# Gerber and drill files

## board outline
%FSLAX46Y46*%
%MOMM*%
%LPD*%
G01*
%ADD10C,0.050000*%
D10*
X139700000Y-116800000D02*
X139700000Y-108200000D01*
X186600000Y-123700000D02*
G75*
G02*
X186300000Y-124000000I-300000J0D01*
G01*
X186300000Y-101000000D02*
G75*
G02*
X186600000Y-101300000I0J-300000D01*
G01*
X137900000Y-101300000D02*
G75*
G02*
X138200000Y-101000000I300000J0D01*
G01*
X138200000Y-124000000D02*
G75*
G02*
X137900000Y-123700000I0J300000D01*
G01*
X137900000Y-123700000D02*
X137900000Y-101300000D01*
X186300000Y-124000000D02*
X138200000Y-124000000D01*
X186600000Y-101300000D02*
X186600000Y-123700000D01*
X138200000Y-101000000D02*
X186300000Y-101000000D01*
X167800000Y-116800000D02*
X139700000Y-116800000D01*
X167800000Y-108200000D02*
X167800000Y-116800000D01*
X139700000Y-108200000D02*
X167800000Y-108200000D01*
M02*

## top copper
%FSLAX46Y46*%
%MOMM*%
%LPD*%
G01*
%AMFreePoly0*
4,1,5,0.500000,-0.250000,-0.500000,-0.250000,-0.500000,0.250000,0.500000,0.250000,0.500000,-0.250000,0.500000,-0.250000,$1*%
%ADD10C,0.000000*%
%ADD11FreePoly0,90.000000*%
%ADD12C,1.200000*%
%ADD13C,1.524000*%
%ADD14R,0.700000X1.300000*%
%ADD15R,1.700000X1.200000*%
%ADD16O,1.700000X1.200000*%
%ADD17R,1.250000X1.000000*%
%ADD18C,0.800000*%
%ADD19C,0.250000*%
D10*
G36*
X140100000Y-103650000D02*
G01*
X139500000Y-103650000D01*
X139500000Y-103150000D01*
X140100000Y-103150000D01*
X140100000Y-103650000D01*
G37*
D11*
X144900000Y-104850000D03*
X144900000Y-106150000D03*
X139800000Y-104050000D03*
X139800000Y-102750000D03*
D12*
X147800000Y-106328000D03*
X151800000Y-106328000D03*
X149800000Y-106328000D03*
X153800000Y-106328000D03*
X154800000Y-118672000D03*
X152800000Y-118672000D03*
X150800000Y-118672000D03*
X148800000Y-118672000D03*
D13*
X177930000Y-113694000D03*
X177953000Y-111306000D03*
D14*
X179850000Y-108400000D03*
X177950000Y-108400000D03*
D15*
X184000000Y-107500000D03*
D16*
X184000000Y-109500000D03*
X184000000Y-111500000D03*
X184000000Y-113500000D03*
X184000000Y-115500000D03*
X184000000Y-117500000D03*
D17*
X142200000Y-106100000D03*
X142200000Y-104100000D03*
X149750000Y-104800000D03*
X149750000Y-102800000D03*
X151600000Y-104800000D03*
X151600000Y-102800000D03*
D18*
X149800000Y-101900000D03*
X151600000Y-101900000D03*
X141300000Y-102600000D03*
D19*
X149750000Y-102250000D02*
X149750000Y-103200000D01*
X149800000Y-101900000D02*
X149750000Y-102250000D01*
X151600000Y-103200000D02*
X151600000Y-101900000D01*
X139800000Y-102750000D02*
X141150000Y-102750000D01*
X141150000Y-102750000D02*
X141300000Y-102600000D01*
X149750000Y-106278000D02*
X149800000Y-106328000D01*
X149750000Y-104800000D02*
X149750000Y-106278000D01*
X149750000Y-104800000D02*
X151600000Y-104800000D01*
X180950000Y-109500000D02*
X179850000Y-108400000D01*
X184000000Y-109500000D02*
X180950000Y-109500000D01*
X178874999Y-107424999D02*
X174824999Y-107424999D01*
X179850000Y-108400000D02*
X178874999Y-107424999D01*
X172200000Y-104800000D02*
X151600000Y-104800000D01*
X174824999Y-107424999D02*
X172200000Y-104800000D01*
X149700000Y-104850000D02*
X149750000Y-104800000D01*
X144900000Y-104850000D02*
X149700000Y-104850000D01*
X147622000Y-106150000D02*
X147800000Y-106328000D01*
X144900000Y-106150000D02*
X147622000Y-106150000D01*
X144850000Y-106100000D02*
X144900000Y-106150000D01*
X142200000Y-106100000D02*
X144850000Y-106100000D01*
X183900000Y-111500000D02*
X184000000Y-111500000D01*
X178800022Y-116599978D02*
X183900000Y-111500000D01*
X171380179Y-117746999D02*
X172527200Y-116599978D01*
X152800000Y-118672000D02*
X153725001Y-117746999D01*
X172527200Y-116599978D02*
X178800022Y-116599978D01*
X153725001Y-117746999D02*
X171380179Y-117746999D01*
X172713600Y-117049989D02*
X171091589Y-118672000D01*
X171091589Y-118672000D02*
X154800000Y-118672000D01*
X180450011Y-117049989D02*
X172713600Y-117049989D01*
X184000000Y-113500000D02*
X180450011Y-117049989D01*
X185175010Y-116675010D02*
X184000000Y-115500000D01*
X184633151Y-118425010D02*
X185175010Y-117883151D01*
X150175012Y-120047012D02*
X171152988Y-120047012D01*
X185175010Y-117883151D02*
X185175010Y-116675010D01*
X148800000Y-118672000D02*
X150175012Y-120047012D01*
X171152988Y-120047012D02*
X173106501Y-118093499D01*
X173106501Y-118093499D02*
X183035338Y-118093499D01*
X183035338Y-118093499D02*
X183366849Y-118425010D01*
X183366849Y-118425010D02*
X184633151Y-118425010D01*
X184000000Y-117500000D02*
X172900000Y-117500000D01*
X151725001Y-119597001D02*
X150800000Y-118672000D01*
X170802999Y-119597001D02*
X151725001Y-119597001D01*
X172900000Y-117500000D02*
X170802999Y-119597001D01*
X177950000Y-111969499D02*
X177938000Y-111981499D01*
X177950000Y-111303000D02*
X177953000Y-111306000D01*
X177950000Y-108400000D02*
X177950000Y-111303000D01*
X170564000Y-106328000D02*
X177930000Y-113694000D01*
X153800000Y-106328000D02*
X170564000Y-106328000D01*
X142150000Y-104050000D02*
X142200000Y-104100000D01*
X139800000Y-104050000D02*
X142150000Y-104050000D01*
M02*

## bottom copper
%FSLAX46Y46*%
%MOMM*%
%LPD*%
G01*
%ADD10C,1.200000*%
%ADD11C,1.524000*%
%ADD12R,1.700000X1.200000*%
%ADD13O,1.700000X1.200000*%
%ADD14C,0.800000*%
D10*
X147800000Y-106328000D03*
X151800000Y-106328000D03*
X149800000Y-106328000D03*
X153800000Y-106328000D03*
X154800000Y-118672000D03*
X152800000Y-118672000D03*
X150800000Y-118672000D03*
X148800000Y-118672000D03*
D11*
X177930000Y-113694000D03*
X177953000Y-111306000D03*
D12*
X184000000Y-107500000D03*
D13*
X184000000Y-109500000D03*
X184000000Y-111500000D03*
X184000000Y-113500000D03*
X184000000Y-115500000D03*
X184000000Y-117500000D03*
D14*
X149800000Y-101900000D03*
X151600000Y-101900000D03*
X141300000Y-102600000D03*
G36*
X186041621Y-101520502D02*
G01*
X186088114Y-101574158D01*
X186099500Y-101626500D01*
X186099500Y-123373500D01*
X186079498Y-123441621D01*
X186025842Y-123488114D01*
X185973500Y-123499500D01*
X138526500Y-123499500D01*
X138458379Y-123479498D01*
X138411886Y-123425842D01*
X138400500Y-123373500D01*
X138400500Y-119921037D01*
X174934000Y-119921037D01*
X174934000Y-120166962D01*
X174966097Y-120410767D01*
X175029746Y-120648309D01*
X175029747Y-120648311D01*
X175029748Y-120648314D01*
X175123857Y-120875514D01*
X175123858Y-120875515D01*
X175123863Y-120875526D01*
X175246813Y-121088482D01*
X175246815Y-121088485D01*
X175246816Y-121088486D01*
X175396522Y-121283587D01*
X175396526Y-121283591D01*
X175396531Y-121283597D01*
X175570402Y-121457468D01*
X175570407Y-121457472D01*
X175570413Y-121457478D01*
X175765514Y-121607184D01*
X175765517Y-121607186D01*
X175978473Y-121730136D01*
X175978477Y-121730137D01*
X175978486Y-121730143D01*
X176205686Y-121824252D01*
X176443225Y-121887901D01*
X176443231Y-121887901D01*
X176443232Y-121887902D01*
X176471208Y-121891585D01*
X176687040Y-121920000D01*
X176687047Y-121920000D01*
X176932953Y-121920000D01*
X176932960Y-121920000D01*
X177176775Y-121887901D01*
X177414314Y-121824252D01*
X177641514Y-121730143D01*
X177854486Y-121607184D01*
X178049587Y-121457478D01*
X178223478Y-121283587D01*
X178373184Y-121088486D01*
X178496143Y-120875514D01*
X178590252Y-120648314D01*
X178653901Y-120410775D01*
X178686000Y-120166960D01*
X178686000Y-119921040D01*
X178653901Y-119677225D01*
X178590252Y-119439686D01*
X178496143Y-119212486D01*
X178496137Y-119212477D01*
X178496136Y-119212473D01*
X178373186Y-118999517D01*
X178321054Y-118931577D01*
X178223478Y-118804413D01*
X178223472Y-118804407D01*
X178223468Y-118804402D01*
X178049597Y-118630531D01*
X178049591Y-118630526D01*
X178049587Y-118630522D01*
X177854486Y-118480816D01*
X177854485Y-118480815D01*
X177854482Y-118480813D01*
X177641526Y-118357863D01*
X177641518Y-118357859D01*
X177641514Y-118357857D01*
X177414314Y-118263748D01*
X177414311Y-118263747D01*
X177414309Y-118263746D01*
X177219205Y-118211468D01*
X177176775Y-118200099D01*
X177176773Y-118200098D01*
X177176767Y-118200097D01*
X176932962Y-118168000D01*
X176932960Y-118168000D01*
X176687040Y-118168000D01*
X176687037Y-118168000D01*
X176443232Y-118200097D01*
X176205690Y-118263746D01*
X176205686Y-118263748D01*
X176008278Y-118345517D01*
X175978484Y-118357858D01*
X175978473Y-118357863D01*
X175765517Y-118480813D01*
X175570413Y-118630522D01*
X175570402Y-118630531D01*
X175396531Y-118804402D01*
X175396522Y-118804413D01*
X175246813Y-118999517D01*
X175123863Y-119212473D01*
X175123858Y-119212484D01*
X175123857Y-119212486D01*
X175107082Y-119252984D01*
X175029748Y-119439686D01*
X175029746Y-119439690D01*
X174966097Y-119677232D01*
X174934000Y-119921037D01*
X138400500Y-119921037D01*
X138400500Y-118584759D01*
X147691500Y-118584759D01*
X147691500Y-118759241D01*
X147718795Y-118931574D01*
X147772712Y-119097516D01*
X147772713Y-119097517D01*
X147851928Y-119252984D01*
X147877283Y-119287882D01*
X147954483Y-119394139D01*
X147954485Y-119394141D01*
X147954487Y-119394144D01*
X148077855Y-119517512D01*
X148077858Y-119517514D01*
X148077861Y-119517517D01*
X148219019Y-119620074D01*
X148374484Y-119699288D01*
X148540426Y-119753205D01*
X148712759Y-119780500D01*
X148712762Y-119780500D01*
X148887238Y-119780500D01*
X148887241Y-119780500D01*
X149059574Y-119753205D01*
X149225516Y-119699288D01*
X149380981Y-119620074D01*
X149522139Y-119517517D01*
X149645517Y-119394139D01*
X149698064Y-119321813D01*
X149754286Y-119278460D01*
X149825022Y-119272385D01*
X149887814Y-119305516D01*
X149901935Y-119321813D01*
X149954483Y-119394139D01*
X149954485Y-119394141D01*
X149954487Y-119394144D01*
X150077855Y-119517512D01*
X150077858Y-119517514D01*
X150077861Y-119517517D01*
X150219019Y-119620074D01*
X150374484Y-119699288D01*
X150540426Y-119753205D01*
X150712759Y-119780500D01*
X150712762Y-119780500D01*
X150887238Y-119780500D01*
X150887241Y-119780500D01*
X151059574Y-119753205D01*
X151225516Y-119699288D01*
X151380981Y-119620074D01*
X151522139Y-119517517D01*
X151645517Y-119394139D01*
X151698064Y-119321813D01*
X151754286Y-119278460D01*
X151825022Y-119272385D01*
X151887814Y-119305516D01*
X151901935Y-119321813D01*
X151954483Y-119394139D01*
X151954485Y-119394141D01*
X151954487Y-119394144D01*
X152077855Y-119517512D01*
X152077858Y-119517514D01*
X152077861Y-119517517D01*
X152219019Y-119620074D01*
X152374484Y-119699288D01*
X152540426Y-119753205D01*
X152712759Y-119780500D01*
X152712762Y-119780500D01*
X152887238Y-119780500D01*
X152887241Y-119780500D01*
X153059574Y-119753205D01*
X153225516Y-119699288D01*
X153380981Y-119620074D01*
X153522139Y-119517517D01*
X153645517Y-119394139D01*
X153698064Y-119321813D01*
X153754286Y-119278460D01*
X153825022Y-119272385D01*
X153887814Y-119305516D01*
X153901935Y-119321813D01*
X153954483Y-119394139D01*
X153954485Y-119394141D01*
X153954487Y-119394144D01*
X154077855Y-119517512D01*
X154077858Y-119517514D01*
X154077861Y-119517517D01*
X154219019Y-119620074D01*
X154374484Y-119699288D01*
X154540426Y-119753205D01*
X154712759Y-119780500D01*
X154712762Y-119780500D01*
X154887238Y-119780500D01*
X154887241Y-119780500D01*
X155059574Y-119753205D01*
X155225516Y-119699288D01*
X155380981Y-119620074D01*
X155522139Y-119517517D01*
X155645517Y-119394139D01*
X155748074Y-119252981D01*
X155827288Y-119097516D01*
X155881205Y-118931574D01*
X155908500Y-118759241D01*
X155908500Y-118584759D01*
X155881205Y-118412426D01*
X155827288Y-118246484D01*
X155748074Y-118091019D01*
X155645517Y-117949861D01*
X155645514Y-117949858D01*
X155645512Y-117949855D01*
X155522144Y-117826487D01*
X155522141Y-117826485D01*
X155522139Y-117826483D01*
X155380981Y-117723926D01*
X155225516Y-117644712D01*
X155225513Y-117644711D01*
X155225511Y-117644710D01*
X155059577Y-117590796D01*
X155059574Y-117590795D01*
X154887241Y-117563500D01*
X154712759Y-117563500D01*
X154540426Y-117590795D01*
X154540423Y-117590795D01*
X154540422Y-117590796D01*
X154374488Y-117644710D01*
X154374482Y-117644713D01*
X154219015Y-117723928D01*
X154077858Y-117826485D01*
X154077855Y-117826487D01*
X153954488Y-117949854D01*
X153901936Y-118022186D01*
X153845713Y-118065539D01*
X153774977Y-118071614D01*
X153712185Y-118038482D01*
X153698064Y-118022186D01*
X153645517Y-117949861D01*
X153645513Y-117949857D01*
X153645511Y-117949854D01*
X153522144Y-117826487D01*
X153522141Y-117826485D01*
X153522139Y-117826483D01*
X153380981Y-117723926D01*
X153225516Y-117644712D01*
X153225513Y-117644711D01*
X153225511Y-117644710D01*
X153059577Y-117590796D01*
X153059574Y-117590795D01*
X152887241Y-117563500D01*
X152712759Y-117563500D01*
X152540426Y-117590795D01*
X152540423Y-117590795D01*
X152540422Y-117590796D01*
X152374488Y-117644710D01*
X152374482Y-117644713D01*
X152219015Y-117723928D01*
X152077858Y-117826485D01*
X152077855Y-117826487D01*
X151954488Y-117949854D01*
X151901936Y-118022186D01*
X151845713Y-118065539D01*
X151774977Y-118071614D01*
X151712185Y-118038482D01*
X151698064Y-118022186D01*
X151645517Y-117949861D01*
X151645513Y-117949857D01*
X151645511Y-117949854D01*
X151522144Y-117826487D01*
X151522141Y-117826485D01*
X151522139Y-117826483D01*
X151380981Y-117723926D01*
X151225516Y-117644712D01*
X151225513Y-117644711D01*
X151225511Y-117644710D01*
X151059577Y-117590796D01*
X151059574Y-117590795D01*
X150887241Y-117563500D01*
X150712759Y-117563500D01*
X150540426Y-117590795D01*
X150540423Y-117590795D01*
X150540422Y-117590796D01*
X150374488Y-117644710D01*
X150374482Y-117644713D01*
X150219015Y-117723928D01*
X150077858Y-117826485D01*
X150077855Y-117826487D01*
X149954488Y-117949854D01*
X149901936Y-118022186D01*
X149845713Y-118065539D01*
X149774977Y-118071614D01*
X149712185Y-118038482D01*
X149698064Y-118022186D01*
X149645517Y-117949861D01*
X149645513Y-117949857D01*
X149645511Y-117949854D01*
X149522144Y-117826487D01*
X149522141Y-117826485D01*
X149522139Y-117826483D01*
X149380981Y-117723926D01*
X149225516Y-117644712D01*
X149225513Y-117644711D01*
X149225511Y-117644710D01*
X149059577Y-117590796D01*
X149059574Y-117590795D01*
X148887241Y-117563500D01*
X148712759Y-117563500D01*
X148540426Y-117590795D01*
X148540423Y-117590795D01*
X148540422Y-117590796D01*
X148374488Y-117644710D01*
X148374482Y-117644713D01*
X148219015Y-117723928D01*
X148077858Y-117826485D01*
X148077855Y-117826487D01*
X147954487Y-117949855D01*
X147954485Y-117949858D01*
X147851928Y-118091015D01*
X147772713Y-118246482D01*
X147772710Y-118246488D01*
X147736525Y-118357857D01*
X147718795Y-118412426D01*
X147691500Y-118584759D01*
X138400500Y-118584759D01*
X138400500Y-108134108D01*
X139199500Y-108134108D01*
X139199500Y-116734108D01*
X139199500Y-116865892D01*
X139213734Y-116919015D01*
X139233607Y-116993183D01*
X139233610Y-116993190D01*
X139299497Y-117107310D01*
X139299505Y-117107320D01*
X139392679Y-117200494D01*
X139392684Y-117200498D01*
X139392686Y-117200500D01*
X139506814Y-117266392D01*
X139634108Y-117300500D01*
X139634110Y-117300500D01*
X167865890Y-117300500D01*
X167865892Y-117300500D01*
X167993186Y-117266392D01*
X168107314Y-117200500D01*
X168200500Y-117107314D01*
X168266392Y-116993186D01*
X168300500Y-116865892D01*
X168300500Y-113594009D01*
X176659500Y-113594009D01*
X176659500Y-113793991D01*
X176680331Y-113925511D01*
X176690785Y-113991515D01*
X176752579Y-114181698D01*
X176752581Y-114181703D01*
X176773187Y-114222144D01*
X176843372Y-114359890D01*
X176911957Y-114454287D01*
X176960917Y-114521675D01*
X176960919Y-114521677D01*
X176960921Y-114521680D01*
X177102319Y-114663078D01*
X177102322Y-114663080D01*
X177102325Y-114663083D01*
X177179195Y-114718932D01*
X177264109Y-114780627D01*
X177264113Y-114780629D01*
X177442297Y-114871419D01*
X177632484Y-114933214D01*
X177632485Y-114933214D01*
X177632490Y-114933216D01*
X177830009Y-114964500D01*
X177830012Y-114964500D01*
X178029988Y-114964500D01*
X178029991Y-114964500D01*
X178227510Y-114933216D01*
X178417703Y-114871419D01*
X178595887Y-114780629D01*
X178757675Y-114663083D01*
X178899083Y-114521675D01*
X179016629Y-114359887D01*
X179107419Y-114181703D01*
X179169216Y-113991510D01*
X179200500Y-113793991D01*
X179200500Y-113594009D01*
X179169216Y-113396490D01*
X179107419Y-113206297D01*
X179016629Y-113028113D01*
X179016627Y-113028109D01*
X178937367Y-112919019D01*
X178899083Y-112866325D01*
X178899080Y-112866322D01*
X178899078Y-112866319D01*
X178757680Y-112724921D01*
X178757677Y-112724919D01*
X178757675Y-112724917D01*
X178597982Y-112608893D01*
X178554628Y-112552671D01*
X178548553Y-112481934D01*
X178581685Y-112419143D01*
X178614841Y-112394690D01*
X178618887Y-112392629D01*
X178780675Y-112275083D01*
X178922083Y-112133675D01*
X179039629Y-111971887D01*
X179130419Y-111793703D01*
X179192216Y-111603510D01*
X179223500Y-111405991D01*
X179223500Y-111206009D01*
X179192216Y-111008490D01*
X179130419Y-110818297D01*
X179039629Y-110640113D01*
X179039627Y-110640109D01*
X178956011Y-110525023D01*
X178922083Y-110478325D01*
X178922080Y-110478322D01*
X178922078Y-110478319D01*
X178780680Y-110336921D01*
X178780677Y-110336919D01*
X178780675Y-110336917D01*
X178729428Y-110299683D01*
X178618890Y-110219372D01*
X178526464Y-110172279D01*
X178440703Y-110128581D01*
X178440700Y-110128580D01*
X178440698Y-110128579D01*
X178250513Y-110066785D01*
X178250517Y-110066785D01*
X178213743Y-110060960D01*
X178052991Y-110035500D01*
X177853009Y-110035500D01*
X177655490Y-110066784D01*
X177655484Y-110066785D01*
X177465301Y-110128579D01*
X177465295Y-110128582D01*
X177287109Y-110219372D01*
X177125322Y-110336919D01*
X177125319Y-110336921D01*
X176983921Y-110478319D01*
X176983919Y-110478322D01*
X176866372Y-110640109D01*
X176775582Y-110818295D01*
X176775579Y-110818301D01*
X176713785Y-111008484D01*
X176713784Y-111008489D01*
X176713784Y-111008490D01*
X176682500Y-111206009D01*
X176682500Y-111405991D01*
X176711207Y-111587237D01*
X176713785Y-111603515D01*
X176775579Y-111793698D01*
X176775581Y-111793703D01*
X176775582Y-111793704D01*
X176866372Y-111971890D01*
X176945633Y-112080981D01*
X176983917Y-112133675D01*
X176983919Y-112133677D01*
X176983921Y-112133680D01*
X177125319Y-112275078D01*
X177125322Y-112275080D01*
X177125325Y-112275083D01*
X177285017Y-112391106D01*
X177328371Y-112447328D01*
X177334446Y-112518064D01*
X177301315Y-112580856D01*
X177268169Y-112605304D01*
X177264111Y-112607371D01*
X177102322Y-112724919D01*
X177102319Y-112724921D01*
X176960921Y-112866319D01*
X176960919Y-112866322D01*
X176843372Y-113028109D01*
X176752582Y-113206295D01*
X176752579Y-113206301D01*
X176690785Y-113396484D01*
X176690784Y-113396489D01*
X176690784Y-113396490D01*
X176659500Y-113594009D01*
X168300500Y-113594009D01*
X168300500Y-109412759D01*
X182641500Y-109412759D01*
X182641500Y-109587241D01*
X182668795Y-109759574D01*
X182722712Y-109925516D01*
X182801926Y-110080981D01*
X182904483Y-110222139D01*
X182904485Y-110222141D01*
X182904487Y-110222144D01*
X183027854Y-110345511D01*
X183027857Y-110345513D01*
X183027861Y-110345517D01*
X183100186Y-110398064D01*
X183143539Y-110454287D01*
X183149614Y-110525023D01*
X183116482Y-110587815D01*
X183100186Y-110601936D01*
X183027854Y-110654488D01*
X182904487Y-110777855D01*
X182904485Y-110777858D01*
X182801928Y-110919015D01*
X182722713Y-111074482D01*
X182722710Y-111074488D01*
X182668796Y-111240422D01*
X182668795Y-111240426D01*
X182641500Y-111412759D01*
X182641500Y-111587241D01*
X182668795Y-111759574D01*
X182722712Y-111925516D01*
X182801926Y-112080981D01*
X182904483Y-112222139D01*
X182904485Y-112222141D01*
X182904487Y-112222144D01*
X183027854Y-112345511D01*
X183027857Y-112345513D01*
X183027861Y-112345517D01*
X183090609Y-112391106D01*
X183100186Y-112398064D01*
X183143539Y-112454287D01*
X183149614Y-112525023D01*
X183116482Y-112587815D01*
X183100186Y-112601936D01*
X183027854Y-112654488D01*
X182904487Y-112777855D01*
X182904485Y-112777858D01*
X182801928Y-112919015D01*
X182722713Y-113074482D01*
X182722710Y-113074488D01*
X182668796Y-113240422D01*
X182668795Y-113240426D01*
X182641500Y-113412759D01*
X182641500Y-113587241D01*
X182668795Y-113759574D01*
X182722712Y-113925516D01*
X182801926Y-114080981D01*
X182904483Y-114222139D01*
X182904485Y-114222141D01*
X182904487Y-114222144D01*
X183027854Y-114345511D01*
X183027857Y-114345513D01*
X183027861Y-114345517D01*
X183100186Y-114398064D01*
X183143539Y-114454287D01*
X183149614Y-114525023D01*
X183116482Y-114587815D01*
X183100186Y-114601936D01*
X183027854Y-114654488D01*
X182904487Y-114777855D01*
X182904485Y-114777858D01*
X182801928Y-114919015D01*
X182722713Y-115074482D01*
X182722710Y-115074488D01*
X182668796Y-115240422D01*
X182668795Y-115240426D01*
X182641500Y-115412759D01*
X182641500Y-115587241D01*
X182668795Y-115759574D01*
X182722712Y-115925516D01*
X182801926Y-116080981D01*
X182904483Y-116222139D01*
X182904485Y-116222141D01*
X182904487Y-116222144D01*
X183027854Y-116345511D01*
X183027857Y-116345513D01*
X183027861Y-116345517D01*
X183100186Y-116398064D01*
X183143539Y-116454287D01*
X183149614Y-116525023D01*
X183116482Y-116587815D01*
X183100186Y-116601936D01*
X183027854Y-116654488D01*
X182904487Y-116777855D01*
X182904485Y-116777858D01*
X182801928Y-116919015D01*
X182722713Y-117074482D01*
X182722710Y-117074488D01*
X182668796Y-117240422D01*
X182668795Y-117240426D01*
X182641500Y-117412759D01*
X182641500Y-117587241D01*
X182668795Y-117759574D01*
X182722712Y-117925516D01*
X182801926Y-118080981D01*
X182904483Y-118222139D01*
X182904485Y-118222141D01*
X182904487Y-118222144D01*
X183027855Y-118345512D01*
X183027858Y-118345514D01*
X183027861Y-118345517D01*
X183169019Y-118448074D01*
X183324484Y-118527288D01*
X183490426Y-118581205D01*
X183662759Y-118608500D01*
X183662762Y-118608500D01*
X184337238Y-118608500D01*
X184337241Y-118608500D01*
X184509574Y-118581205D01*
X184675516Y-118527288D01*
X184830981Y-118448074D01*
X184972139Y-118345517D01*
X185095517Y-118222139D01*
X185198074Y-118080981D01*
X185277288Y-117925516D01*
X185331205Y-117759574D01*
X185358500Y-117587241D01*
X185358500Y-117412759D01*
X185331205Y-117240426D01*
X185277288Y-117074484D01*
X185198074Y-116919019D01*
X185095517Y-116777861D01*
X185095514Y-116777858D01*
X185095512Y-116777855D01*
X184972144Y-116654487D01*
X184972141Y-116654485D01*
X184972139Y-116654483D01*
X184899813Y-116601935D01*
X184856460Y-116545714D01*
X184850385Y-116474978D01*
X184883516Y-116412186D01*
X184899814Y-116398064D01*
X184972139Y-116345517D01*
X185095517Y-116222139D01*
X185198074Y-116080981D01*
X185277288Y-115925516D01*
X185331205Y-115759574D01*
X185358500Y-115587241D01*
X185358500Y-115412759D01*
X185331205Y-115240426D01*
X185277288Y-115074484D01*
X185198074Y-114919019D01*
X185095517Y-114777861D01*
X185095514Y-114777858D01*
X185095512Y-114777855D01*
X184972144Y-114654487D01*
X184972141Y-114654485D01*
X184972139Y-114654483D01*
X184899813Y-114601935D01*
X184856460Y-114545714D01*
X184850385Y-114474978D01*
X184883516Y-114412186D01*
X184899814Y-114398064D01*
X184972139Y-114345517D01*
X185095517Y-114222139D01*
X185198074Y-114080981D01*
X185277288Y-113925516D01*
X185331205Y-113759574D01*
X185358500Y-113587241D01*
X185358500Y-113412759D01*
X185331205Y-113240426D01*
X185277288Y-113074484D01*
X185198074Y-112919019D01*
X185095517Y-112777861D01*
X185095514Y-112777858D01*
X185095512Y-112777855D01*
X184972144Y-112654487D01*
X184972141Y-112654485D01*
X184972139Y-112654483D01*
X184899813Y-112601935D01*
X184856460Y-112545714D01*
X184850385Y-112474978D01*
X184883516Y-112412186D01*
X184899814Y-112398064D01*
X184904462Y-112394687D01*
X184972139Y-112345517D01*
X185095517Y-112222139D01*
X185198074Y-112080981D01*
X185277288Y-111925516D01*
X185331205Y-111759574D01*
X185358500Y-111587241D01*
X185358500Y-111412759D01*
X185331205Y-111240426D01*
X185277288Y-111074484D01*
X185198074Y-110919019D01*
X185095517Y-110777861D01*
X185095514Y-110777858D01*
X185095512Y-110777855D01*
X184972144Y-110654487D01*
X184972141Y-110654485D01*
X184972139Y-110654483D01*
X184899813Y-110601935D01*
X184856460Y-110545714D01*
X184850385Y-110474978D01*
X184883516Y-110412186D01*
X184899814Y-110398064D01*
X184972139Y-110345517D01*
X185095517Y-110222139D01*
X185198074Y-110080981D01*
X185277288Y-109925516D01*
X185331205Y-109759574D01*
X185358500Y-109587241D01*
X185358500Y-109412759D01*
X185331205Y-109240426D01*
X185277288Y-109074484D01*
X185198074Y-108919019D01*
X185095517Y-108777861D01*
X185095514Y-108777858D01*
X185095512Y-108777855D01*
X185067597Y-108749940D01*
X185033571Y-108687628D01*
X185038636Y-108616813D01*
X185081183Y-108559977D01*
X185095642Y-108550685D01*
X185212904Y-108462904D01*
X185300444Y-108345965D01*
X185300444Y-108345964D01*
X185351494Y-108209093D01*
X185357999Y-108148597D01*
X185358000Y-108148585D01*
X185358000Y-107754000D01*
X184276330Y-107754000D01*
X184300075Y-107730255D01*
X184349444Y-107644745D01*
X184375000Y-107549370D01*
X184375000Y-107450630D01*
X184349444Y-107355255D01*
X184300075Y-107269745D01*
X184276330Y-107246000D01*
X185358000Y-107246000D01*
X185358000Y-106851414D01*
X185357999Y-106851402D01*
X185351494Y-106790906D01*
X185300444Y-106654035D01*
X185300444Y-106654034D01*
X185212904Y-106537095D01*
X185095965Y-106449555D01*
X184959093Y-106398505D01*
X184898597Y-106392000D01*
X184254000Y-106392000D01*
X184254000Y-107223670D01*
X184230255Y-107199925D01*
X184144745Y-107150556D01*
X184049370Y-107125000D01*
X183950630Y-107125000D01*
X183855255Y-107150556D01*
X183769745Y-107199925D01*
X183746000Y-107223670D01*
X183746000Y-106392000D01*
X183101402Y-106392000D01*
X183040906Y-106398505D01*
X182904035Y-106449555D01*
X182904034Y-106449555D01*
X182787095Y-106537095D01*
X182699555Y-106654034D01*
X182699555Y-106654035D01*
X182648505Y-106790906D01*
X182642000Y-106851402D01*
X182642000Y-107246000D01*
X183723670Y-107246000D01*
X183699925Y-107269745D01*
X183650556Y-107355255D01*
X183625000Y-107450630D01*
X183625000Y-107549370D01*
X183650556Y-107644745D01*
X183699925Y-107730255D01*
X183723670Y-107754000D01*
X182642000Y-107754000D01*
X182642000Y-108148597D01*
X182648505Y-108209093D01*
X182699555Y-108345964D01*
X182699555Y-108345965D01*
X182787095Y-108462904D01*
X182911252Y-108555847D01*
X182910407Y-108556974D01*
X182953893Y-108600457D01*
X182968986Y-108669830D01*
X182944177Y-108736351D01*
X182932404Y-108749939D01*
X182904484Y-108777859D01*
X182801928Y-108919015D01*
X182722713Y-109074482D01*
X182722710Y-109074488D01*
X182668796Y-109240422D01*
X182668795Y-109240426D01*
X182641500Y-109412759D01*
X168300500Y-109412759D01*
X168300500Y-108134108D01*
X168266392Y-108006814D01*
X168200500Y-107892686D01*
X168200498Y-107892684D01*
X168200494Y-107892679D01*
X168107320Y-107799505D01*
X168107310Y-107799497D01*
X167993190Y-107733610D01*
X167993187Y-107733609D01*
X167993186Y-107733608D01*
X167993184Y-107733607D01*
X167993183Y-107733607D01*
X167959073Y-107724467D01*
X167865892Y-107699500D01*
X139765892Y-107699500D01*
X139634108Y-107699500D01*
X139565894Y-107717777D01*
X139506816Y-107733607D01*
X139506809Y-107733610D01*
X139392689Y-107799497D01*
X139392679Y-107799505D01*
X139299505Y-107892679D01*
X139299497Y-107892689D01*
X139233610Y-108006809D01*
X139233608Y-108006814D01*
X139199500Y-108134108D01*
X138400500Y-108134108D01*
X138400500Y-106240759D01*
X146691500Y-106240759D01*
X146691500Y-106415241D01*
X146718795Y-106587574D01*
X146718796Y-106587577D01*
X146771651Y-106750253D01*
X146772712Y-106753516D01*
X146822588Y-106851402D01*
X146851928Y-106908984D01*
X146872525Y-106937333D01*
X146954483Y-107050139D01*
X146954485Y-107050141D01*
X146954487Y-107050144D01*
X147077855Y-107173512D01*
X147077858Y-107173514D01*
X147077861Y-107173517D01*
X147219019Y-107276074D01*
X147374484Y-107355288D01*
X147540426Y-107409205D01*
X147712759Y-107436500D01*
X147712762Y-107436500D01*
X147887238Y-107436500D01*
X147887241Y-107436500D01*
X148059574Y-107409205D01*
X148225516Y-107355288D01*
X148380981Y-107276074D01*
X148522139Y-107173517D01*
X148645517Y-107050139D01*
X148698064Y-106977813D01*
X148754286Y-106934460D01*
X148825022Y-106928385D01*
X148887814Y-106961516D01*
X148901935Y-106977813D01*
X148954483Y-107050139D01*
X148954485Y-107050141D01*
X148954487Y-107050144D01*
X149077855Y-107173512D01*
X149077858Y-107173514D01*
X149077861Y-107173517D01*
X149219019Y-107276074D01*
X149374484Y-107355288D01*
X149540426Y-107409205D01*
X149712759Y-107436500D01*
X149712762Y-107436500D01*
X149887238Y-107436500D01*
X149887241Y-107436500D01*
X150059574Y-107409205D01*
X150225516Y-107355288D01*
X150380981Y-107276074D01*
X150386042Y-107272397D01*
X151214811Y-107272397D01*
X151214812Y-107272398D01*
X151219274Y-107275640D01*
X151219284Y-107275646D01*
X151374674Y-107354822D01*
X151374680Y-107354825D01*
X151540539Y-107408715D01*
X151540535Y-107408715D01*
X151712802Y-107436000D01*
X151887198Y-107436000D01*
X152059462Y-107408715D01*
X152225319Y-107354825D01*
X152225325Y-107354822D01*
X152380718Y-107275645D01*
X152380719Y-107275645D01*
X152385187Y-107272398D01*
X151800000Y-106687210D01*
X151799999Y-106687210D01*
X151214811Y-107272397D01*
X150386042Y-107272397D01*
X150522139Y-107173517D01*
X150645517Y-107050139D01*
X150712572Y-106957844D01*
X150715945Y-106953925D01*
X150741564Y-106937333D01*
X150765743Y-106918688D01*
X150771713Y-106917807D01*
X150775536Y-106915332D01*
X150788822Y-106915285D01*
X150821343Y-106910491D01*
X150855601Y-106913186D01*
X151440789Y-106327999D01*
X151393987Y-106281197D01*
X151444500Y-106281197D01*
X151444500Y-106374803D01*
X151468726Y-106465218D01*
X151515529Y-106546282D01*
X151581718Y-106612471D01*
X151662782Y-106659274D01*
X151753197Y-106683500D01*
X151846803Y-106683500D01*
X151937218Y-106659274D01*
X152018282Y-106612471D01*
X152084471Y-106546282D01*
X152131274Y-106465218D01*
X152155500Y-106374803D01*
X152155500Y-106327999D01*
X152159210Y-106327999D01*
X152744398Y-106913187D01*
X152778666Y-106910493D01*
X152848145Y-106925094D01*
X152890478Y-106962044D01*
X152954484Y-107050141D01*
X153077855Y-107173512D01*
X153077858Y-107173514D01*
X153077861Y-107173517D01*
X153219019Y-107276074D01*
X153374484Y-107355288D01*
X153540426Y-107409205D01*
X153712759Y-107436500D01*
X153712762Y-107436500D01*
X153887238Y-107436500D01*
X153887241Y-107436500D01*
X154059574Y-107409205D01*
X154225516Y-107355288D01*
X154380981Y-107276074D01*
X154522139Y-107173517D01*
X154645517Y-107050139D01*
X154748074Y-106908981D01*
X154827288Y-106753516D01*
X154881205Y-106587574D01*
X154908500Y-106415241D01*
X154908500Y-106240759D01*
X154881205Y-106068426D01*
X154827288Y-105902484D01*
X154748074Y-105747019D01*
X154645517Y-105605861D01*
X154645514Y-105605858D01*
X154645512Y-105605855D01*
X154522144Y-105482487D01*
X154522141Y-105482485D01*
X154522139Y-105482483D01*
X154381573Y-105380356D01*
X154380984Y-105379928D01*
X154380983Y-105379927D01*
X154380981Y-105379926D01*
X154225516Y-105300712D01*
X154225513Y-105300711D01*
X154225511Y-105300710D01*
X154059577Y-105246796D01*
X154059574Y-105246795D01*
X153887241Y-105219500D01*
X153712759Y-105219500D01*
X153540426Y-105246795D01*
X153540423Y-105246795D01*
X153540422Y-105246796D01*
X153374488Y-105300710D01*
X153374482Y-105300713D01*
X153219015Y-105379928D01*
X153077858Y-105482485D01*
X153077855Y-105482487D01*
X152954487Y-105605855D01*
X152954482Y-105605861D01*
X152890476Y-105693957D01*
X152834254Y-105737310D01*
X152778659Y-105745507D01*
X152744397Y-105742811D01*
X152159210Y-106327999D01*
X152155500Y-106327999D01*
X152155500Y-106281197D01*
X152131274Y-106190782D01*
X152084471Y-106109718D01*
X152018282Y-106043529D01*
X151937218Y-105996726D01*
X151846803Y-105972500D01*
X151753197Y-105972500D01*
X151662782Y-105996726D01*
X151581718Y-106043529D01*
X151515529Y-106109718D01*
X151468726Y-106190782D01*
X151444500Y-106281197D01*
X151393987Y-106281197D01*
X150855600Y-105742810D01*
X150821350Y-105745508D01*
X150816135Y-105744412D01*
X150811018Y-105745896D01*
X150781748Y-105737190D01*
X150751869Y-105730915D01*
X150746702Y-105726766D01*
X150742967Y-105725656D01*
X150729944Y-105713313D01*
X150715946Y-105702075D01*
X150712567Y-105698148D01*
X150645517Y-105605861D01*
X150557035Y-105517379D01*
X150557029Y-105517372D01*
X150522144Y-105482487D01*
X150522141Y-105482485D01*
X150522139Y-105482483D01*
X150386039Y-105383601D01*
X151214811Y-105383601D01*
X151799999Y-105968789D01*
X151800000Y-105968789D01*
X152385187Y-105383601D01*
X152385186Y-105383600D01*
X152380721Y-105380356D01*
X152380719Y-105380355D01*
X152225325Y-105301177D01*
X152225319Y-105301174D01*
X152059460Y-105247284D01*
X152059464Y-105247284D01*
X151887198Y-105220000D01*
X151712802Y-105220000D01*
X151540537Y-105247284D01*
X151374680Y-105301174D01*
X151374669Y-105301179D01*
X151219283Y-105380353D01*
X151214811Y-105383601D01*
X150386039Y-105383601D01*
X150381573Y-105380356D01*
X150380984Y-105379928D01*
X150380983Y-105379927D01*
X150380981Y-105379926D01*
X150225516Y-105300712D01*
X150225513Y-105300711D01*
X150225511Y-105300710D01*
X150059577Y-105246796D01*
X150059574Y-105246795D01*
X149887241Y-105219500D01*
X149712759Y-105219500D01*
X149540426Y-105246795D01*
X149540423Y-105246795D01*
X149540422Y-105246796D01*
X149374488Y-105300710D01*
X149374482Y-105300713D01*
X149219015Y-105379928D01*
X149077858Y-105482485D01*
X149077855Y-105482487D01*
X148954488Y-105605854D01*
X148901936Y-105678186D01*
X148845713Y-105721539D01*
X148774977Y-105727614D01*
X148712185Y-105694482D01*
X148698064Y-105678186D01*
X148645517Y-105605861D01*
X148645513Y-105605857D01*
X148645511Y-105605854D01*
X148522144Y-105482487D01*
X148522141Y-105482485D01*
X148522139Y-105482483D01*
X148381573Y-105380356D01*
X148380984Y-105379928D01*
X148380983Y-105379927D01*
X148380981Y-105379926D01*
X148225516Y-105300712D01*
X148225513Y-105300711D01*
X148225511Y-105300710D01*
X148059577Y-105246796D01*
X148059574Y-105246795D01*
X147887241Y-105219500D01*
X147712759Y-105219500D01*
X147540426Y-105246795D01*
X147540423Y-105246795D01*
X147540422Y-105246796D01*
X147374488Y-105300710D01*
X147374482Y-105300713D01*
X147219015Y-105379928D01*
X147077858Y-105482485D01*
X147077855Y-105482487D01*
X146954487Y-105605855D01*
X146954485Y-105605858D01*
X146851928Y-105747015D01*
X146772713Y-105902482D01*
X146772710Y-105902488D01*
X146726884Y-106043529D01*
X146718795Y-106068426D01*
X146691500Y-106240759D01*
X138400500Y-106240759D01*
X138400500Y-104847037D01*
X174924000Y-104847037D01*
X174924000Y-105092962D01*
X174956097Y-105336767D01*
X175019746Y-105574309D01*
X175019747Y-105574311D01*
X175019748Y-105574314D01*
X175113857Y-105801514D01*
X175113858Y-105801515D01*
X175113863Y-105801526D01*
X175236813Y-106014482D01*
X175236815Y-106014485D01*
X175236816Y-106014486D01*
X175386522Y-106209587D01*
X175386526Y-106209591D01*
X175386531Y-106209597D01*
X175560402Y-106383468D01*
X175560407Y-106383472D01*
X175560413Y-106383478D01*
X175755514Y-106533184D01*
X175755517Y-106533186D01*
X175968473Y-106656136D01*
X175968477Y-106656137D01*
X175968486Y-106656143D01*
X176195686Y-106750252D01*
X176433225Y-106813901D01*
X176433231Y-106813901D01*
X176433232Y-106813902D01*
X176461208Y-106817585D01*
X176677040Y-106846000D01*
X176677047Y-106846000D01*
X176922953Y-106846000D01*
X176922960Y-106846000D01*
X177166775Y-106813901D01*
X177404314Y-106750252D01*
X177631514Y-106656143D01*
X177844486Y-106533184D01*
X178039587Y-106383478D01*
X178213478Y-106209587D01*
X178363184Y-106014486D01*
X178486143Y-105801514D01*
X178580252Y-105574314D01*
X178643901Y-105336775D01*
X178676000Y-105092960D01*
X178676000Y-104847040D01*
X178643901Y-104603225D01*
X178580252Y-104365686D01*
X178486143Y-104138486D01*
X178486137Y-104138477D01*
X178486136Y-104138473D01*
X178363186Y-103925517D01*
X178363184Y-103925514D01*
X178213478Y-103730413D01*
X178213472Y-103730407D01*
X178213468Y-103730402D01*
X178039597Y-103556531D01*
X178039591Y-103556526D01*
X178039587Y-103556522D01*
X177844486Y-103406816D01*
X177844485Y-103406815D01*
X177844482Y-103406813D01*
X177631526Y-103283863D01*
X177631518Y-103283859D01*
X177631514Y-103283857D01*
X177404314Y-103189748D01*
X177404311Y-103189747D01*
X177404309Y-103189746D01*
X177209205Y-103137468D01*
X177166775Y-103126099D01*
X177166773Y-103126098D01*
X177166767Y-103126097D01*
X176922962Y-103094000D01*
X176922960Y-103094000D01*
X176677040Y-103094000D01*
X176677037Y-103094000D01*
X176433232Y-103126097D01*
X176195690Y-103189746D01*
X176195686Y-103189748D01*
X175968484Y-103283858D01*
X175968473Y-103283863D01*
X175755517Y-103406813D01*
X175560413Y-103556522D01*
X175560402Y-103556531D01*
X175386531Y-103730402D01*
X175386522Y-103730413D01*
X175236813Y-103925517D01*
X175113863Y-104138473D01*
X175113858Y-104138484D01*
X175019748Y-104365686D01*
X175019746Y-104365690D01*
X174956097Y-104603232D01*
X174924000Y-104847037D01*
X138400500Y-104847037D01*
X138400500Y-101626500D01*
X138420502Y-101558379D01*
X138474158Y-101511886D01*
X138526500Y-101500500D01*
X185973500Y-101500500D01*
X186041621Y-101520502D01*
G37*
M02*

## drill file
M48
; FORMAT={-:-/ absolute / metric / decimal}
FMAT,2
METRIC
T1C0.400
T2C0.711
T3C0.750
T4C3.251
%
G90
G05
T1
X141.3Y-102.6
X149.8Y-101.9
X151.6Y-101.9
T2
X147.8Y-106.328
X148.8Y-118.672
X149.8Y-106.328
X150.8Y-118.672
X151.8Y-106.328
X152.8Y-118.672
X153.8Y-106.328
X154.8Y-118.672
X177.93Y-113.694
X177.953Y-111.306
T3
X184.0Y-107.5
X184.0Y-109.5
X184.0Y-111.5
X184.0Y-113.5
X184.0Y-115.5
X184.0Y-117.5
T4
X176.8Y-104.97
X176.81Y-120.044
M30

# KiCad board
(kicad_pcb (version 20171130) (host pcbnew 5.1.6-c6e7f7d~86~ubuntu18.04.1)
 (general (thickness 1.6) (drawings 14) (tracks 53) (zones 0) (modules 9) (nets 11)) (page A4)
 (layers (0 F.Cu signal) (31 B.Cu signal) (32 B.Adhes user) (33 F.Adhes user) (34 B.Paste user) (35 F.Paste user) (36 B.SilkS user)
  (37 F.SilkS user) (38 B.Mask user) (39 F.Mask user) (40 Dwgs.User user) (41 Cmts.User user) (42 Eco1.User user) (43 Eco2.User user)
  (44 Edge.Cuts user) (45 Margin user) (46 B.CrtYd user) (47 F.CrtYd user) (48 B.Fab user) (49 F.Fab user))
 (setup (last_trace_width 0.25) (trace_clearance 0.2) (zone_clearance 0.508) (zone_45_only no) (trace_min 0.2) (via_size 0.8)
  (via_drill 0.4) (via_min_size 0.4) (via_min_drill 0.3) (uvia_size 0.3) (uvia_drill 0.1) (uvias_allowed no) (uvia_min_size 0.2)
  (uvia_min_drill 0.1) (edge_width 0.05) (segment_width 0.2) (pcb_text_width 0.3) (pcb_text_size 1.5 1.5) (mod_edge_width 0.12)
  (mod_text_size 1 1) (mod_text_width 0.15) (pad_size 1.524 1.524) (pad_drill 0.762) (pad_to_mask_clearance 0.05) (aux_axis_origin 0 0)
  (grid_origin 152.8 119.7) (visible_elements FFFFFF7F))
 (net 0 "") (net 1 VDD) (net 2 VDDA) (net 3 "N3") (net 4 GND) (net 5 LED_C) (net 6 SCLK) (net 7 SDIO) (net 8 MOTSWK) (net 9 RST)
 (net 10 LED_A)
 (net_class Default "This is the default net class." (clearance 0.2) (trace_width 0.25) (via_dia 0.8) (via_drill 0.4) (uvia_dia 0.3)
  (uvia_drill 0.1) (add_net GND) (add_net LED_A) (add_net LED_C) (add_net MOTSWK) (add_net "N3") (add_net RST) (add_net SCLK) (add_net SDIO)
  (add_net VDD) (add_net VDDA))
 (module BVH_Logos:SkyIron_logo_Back (layer F.Cu) (at 175.6 111.7)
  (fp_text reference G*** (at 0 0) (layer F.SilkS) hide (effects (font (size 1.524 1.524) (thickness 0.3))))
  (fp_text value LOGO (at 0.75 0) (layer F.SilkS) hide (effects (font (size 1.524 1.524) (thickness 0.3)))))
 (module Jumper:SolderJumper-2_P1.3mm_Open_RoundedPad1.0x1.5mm (layer F.Cu) (at 144.9 105.5 90)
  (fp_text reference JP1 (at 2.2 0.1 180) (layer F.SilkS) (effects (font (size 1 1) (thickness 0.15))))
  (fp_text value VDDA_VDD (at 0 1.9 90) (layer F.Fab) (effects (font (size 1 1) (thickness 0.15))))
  (pad 2 smd custom (at 0.65 0 90) (size 1 0.5) (layers F.Cu F.Mask) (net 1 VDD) (zone_connect 2)
   (options (clearance outline) (anchor rect)) (primitives))
  (pad 1 smd custom (at -0.65 0 90) (size 1 0.5) (layers F.Cu F.Mask) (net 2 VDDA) (zone_connect 2)
   (options (clearance outline) (anchor rect)) (primitives)))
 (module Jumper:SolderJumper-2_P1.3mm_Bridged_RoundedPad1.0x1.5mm (layer F.Cu) (at 139.8 103.4 90)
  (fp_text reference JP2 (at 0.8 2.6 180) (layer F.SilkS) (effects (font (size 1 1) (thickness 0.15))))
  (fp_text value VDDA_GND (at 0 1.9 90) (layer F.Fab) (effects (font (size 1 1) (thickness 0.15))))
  (fp_poly (pts (xy 0.25 -0.3) (xy -0.25 -0.3) (xy -0.25 0.3) (xy 0.25 0.3)) (layer F.Cu) (width 0))
  (pad 1 smd custom (at -0.65 0 90) (size 1 0.5) (layers F.Cu F.Mask) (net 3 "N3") (zone_connect 2)
   (options (clearance outline) (anchor rect)) (primitives))
  (pad 2 smd custom (at 0.65 0 90) (size 1 0.5) (layers F.Cu F.Mask) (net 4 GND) (zone_connect 2)
   (options (clearance outline) (anchor rect)) (primitives)))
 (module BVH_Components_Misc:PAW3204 (layer F.Cu) (at 150.8 112.5)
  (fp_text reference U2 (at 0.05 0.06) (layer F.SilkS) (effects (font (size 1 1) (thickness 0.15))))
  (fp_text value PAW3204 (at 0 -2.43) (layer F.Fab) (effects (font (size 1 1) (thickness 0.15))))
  (pad 8 thru_hole circle (at -3 -6.172 180) (size 1.2 1.2) (drill 0.711) (layers *.Cu *.Mask) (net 2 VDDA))
  (pad 6 thru_hole circle (at 1 -6.172 180) (size 1.2 1.2) (drill 0.711) (layers *.Cu *.Mask) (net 4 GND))
  (pad 7 thru_hole circle (at -1 -6.172 180) (size 1.2 1.2) (drill 0.711) (layers *.Cu *.Mask) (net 1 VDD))
  (pad 5 thru_hole circle (at 3 -6.172 180) (size 1.2 1.2) (drill 0.711) (layers *.Cu *.Mask) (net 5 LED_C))
  (pad 4 thru_hole circle (at 4 6.172) (size 1.2 1.2) (drill 0.711) (layers *.Cu *.Mask) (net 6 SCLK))
  (pad 3 thru_hole circle (at 2 6.172) (size 1.2 1.2) (drill 0.711) (layers *.Cu *.Mask) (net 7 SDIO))
  (pad 2 thru_hole circle (at 0 6.172) (size 1.2 1.2) (drill 0.711) (layers *.Cu *.Mask) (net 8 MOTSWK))
  (pad 1 thru_hole circle (at -2 6.172) (size 1.2 1.2) (drill 0.711) (layers *.Cu *.Mask) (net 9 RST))
  (pad "" np_thru_hole circle (at 26 -7.53) (size 3.251 3.251) (drill 3.251) (layers *.Cu *.Mask))
  (pad "" np_thru_hole circle (at 26.01 7.544) (size 3.251 3.251) (drill 3.251) (layers *.Cu *.Mask))
  (pad 10 thru_hole circle (at 27.13 1.194) (size 1.524 1.524) (drill 0.711) (layers *.Cu *.Mask) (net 5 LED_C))
  (pad 9 thru_hole circle (at 27.153 -1.194) (size 1.524 1.524) (drill 0.711) (layers *.Cu *.Mask) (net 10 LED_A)))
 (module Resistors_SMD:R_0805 (layer F.Cu) (at 178.9 108.4 180)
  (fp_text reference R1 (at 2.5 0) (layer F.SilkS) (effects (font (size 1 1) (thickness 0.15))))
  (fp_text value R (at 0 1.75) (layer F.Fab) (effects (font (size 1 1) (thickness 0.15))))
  (pad 1 smd rect (at -0.95 0 180) (size 0.7 1.3) (layers F.Cu F.Paste F.Mask) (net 1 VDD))
  (pad 2 smd rect (at 0.95 0 180) (size 0.7 1.3) (layers F.Cu F.Paste F.Mask) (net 10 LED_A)))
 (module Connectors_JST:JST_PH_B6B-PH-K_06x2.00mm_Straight (layer F.Cu) (at 184 107.5 270)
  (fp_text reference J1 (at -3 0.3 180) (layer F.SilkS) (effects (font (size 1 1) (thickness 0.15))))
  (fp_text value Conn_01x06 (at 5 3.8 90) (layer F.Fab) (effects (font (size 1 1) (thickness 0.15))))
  (pad 1 thru_hole rect (at 0 0 270) (size 1.2 1.7) (drill 0.75) (layers *.Cu *.Mask) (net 4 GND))
  (pad 2 thru_hole oval (at 2 0 270) (size 1.2 1.7) (drill 0.75) (layers *.Cu *.Mask) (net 1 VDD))
  (pad 3 thru_hole oval (at 4 0 270) (size 1.2 1.7) (drill 0.75) (layers *.Cu *.Mask) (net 7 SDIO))
  (pad 4 thru_hole oval (at 6 0 270) (size 1.2 1.7) (drill 0.75) (layers *.Cu *.Mask) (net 6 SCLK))
  (pad 5 thru_hole oval (at 8 0 270) (size 1.2 1.7) (drill 0.75) (layers *.Cu *.Mask) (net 9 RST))
  (pad 6 thru_hole oval (at 10 0 270) (size 1.2 1.7) (drill 0.75) (layers *.Cu *.Mask) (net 8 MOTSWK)))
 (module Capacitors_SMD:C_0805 (layer F.Cu) (at 142.2 105.1 90)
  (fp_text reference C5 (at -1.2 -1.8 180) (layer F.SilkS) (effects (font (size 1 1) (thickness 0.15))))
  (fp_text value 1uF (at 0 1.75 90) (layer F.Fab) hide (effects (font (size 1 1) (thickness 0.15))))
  (pad 1 smd rect (at -1 0 90) (size 1 1.25) (layers F.Cu F.Paste F.Mask) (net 2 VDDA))
  (pad 2 smd rect (at 1 0 90) (size 1 1.25) (layers F.Cu F.Paste F.Mask) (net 3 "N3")))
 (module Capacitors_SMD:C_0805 (layer F.Cu) (at 149.75 103.8 90)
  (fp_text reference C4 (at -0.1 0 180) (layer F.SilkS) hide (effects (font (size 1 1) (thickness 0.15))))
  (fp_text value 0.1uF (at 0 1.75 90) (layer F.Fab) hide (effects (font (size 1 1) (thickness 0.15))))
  (pad 1 smd rect (at -1 0 90) (size 1 1.25) (layers F.Cu F.Paste F.Mask) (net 1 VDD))
  (pad 2 smd rect (at 1 0 90) (size 1 1.25) (layers F.Cu F.Paste F.Mask) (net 4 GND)))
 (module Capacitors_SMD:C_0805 (layer F.Cu) (at 151.6 103.8 90)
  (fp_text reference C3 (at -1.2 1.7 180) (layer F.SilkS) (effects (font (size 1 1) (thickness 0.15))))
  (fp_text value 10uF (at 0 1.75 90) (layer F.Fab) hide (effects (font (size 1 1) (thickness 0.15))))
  (pad 1 smd rect (at -1 0 90) (size 1 1.25) (layers F.Cu F.Paste F.Mask) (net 1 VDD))
  (pad 2 smd rect (at 1 0 90) (size 1 1.25) (layers F.Cu F.Paste F.Mask) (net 4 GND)))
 (gr_line (start 139.7 116.8) (end 139.7 108.2) (layer Edge.Cuts) (width 0.05))
 (gr_arc (start 186.3 123.7) (end 186.3 124) (angle -90) (layer Edge.Cuts) (width 0.05))
 (gr_arc (start 186.3 101.3) (end 186.6 101.3) (angle -90) (layer Edge.Cuts) (width 0.05))
 (gr_arc (start 138.2 101.3) (end 138.2 101) (angle -90) (layer Edge.Cuts) (width 0.05))
 (gr_arc (start 138.2 123.7) (end 137.9 123.7) (angle -90) (layer Edge.Cuts) (width 0.05))
 (gr_line (start 137.9 123.7) (end 137.9 101.3) (layer Edge.Cuts) (width 0.05))
 (gr_line (start 186.3 124) (end 138.2 124) (layer Edge.Cuts) (width 0.05))
 (gr_line (start 186.6 101.3) (end 186.6 123.7) (layer Edge.Cuts) (width 0.05))
 (gr_line (start 138.2 101) (end 186.3 101) (layer Edge.Cuts) (width 0.05))
 (gr_line (start 167.8 116.8) (end 139.7 116.8) (layer Edge.Cuts) (width 0.05))
 (gr_line (start 167.8 108.2) (end 167.8 116.8) (layer Edge.Cuts) (width 0.05))
 (gr_line (start 139.7 108.2) (end 167.8 108.2) (layer Edge.Cuts) (width 0.05))
 (via (at 149.8 101.9) (size 0.8) (drill 0.4) (layers F.Cu B.Cu) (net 4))
 (segment (start 149.75 102.25) (end 149.75 103.2) (width 0.25) (layer F.Cu) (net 4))
 (segment (start 149.8 101.9) (end 149.75 102.25) (width 0.25) (layer F.Cu) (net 4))
 (segment (start 151.6 103.2) (end 151.6 101.9) (width 0.25) (layer F.Cu) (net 4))
 (via (at 151.6 101.9) (size 0.8) (drill 0.4) (layers F.Cu B.Cu) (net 4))
 (via (at 141.3 102.6) (size 0.8) (drill 0.4) (layers F.Cu B.Cu) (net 4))
 (segment (start 139.8 102.75) (end 141.15 102.75) (width 0.25) (layer F.Cu) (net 4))
 (segment (start 141.15 102.75) (end 141.3 102.6) (width 0.25) (layer F.Cu) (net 4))
 (segment (start 149.75 106.278) (end 149.8 106.328) (width 0.25) (layer F.Cu) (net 1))
 (segment (start 149.75 104.8) (end 149.75 106.278) (width 0.25) (layer F.Cu) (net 1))
 (segment (start 149.75 104.8) (end 151.6 104.8) (width 0.25) (layer F.Cu) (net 1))
 (segment (start 180.95 109.5) (end 179.85 108.4) (width 0.25) (layer F.Cu) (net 1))
 (segment (start 184 109.5) (end 180.95 109.5) (width 0.25) (layer F.Cu) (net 1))
 (segment (start 178.874999 107.424999) (end 174.824999 107.424999) (width 0.25) (layer F.Cu) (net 1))
 (segment (start 179.85 108.4) (end 178.874999 107.424999) (width 0.25) (layer F.Cu) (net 1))
 (segment (start 172.2 104.8) (end 151.6 104.8) (width 0.25) (layer F.Cu) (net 1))
 (segment (start 174.824999 107.424999) (end 172.2 104.8) (width 0.25) (layer F.Cu) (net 1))
 (segment (start 149.7 104.85) (end 149.75 104.8) (width 0.25) (layer F.Cu) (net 1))
 (segment (start 144.9 104.85) (end 149.7 104.85) (width 0.25) (layer F.Cu) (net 1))
 (segment (start 147.622 106.15) (end 147.8 106.328) (width 0.25) (layer F.Cu) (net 2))
 (segment (start 144.9 106.15) (end 147.622 106.15) (width 0.25) (layer F.Cu) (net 2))
 (segment (start 144.85 106.1) (end 144.9 106.15) (width 0.25) (layer F.Cu) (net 2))
 (segment (start 142.2 106.1) (end 144.85 106.1) (width 0.25) (layer F.Cu) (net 2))
 (segment (start 183.9 111.5) (end 184 111.5) (width 0.25) (layer F.Cu) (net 7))
 (segment (start 178.800022 116.599978) (end 183.9 111.5) (width 0.25) (layer F.Cu) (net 7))
 (segment (start 171.380179 117.746999) (end 172.5272 116.599978) (width 0.25) (layer F.Cu) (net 7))
 (segment (start 152.8 118.672) (end 153.725001 117.746999) (width 0.25) (layer F.Cu) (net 7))
 (segment (start 172.5272 116.599978) (end 178.800022 116.599978) (width 0.25) (layer F.Cu) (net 7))
 (segment (start 153.725001 117.746999) (end 171.380179 117.746999) (width 0.25) (layer F.Cu) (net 7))
 (segment (start 172.7136 117.049989) (end 171.091589 118.672) (width 0.25) (layer F.Cu) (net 6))
 (segment (start 171.091589 118.672) (end 154.8 118.672) (width 0.25) (layer F.Cu) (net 6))
 (segment (start 180.450011 117.049989) (end 172.7136 117.049989) (width 0.25) (layer F.Cu) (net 6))
 (segment (start 184 113.5) (end 180.450011 117.049989) (width 0.25) (layer F.Cu) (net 6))
 (segment (start 185.17501 116.67501) (end 184 115.5) (width 0.25) (layer F.Cu) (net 9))
 (segment (start 184.633151 118.42501) (end 185.17501 117.883151) (width 0.25) (layer F.Cu) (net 9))
 (segment (start 150.175012 120.047012) (end 171.152988 120.047012) (width 0.25) (layer F.Cu) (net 9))
 (segment (start 185.17501 117.883151) (end 185.17501 116.67501) (width 0.25) (layer F.Cu) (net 9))
 (segment (start 148.8 118.672) (end 150.175012 120.047012) (width 0.25) (layer F.Cu) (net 9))
 (segment (start 171.152988 120.047012) (end 173.106501 118.093499) (width 0.25) (layer F.Cu) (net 9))
 (segment (start 173.106501 118.093499) (end 183.035338 118.093499) (width 0.25) (layer F.Cu) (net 9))
 (segment (start 183.035338 118.093499) (end 183.366849 118.42501) (width 0.25) (layer F.Cu) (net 9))
 (segment (start 183.366849 118.42501) (end 184.633151 118.42501) (width 0.25) (layer F.Cu) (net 9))
 (segment (start 184 117.5) (end 172.9 117.5) (width 0.25) (layer F.Cu) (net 8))
 (segment (start 151.725001 119.597001) (end 150.8 118.672) (width 0.25) (layer F.Cu) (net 8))
 (segment (start 170.802999 119.597001) (end 151.725001 119.597001) (width 0.25) (layer F.Cu) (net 8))
 (segment (start 172.9 117.5) (end 170.802999 119.597001) (width 0.25) (layer F.Cu) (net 8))
 (segment (start 177.95 111.969499) (end 177.938 111.981499) (width 0.25) (layer F.Cu) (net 10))
 (segment (start 177.95 111.303) (end 177.953 111.306) (width 0.25) (layer F.Cu) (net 10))
 (segment (start 177.95 108.4) (end 177.95 111.303) (width 0.25) (layer F.Cu) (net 10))
 (segment (start 170.564 106.328) (end 177.93 113.694) (width 0.25) (layer F.Cu) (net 5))
 (segment (start 153.8 106.328) (end 170.564 106.328) (width 0.25) (layer F.Cu) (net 5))
 (segment (start 142.15 104.05) (end 142.2 104.1) (width 0.25) (layer F.Cu) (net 3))
 (segment (start 139.8 104.05) (end 142.15 104.05) (width 0.25) (layer F.Cu) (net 3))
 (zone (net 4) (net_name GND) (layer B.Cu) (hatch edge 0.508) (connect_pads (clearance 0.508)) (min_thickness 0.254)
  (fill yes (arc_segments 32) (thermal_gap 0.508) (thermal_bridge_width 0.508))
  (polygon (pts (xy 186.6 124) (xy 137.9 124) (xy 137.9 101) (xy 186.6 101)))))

